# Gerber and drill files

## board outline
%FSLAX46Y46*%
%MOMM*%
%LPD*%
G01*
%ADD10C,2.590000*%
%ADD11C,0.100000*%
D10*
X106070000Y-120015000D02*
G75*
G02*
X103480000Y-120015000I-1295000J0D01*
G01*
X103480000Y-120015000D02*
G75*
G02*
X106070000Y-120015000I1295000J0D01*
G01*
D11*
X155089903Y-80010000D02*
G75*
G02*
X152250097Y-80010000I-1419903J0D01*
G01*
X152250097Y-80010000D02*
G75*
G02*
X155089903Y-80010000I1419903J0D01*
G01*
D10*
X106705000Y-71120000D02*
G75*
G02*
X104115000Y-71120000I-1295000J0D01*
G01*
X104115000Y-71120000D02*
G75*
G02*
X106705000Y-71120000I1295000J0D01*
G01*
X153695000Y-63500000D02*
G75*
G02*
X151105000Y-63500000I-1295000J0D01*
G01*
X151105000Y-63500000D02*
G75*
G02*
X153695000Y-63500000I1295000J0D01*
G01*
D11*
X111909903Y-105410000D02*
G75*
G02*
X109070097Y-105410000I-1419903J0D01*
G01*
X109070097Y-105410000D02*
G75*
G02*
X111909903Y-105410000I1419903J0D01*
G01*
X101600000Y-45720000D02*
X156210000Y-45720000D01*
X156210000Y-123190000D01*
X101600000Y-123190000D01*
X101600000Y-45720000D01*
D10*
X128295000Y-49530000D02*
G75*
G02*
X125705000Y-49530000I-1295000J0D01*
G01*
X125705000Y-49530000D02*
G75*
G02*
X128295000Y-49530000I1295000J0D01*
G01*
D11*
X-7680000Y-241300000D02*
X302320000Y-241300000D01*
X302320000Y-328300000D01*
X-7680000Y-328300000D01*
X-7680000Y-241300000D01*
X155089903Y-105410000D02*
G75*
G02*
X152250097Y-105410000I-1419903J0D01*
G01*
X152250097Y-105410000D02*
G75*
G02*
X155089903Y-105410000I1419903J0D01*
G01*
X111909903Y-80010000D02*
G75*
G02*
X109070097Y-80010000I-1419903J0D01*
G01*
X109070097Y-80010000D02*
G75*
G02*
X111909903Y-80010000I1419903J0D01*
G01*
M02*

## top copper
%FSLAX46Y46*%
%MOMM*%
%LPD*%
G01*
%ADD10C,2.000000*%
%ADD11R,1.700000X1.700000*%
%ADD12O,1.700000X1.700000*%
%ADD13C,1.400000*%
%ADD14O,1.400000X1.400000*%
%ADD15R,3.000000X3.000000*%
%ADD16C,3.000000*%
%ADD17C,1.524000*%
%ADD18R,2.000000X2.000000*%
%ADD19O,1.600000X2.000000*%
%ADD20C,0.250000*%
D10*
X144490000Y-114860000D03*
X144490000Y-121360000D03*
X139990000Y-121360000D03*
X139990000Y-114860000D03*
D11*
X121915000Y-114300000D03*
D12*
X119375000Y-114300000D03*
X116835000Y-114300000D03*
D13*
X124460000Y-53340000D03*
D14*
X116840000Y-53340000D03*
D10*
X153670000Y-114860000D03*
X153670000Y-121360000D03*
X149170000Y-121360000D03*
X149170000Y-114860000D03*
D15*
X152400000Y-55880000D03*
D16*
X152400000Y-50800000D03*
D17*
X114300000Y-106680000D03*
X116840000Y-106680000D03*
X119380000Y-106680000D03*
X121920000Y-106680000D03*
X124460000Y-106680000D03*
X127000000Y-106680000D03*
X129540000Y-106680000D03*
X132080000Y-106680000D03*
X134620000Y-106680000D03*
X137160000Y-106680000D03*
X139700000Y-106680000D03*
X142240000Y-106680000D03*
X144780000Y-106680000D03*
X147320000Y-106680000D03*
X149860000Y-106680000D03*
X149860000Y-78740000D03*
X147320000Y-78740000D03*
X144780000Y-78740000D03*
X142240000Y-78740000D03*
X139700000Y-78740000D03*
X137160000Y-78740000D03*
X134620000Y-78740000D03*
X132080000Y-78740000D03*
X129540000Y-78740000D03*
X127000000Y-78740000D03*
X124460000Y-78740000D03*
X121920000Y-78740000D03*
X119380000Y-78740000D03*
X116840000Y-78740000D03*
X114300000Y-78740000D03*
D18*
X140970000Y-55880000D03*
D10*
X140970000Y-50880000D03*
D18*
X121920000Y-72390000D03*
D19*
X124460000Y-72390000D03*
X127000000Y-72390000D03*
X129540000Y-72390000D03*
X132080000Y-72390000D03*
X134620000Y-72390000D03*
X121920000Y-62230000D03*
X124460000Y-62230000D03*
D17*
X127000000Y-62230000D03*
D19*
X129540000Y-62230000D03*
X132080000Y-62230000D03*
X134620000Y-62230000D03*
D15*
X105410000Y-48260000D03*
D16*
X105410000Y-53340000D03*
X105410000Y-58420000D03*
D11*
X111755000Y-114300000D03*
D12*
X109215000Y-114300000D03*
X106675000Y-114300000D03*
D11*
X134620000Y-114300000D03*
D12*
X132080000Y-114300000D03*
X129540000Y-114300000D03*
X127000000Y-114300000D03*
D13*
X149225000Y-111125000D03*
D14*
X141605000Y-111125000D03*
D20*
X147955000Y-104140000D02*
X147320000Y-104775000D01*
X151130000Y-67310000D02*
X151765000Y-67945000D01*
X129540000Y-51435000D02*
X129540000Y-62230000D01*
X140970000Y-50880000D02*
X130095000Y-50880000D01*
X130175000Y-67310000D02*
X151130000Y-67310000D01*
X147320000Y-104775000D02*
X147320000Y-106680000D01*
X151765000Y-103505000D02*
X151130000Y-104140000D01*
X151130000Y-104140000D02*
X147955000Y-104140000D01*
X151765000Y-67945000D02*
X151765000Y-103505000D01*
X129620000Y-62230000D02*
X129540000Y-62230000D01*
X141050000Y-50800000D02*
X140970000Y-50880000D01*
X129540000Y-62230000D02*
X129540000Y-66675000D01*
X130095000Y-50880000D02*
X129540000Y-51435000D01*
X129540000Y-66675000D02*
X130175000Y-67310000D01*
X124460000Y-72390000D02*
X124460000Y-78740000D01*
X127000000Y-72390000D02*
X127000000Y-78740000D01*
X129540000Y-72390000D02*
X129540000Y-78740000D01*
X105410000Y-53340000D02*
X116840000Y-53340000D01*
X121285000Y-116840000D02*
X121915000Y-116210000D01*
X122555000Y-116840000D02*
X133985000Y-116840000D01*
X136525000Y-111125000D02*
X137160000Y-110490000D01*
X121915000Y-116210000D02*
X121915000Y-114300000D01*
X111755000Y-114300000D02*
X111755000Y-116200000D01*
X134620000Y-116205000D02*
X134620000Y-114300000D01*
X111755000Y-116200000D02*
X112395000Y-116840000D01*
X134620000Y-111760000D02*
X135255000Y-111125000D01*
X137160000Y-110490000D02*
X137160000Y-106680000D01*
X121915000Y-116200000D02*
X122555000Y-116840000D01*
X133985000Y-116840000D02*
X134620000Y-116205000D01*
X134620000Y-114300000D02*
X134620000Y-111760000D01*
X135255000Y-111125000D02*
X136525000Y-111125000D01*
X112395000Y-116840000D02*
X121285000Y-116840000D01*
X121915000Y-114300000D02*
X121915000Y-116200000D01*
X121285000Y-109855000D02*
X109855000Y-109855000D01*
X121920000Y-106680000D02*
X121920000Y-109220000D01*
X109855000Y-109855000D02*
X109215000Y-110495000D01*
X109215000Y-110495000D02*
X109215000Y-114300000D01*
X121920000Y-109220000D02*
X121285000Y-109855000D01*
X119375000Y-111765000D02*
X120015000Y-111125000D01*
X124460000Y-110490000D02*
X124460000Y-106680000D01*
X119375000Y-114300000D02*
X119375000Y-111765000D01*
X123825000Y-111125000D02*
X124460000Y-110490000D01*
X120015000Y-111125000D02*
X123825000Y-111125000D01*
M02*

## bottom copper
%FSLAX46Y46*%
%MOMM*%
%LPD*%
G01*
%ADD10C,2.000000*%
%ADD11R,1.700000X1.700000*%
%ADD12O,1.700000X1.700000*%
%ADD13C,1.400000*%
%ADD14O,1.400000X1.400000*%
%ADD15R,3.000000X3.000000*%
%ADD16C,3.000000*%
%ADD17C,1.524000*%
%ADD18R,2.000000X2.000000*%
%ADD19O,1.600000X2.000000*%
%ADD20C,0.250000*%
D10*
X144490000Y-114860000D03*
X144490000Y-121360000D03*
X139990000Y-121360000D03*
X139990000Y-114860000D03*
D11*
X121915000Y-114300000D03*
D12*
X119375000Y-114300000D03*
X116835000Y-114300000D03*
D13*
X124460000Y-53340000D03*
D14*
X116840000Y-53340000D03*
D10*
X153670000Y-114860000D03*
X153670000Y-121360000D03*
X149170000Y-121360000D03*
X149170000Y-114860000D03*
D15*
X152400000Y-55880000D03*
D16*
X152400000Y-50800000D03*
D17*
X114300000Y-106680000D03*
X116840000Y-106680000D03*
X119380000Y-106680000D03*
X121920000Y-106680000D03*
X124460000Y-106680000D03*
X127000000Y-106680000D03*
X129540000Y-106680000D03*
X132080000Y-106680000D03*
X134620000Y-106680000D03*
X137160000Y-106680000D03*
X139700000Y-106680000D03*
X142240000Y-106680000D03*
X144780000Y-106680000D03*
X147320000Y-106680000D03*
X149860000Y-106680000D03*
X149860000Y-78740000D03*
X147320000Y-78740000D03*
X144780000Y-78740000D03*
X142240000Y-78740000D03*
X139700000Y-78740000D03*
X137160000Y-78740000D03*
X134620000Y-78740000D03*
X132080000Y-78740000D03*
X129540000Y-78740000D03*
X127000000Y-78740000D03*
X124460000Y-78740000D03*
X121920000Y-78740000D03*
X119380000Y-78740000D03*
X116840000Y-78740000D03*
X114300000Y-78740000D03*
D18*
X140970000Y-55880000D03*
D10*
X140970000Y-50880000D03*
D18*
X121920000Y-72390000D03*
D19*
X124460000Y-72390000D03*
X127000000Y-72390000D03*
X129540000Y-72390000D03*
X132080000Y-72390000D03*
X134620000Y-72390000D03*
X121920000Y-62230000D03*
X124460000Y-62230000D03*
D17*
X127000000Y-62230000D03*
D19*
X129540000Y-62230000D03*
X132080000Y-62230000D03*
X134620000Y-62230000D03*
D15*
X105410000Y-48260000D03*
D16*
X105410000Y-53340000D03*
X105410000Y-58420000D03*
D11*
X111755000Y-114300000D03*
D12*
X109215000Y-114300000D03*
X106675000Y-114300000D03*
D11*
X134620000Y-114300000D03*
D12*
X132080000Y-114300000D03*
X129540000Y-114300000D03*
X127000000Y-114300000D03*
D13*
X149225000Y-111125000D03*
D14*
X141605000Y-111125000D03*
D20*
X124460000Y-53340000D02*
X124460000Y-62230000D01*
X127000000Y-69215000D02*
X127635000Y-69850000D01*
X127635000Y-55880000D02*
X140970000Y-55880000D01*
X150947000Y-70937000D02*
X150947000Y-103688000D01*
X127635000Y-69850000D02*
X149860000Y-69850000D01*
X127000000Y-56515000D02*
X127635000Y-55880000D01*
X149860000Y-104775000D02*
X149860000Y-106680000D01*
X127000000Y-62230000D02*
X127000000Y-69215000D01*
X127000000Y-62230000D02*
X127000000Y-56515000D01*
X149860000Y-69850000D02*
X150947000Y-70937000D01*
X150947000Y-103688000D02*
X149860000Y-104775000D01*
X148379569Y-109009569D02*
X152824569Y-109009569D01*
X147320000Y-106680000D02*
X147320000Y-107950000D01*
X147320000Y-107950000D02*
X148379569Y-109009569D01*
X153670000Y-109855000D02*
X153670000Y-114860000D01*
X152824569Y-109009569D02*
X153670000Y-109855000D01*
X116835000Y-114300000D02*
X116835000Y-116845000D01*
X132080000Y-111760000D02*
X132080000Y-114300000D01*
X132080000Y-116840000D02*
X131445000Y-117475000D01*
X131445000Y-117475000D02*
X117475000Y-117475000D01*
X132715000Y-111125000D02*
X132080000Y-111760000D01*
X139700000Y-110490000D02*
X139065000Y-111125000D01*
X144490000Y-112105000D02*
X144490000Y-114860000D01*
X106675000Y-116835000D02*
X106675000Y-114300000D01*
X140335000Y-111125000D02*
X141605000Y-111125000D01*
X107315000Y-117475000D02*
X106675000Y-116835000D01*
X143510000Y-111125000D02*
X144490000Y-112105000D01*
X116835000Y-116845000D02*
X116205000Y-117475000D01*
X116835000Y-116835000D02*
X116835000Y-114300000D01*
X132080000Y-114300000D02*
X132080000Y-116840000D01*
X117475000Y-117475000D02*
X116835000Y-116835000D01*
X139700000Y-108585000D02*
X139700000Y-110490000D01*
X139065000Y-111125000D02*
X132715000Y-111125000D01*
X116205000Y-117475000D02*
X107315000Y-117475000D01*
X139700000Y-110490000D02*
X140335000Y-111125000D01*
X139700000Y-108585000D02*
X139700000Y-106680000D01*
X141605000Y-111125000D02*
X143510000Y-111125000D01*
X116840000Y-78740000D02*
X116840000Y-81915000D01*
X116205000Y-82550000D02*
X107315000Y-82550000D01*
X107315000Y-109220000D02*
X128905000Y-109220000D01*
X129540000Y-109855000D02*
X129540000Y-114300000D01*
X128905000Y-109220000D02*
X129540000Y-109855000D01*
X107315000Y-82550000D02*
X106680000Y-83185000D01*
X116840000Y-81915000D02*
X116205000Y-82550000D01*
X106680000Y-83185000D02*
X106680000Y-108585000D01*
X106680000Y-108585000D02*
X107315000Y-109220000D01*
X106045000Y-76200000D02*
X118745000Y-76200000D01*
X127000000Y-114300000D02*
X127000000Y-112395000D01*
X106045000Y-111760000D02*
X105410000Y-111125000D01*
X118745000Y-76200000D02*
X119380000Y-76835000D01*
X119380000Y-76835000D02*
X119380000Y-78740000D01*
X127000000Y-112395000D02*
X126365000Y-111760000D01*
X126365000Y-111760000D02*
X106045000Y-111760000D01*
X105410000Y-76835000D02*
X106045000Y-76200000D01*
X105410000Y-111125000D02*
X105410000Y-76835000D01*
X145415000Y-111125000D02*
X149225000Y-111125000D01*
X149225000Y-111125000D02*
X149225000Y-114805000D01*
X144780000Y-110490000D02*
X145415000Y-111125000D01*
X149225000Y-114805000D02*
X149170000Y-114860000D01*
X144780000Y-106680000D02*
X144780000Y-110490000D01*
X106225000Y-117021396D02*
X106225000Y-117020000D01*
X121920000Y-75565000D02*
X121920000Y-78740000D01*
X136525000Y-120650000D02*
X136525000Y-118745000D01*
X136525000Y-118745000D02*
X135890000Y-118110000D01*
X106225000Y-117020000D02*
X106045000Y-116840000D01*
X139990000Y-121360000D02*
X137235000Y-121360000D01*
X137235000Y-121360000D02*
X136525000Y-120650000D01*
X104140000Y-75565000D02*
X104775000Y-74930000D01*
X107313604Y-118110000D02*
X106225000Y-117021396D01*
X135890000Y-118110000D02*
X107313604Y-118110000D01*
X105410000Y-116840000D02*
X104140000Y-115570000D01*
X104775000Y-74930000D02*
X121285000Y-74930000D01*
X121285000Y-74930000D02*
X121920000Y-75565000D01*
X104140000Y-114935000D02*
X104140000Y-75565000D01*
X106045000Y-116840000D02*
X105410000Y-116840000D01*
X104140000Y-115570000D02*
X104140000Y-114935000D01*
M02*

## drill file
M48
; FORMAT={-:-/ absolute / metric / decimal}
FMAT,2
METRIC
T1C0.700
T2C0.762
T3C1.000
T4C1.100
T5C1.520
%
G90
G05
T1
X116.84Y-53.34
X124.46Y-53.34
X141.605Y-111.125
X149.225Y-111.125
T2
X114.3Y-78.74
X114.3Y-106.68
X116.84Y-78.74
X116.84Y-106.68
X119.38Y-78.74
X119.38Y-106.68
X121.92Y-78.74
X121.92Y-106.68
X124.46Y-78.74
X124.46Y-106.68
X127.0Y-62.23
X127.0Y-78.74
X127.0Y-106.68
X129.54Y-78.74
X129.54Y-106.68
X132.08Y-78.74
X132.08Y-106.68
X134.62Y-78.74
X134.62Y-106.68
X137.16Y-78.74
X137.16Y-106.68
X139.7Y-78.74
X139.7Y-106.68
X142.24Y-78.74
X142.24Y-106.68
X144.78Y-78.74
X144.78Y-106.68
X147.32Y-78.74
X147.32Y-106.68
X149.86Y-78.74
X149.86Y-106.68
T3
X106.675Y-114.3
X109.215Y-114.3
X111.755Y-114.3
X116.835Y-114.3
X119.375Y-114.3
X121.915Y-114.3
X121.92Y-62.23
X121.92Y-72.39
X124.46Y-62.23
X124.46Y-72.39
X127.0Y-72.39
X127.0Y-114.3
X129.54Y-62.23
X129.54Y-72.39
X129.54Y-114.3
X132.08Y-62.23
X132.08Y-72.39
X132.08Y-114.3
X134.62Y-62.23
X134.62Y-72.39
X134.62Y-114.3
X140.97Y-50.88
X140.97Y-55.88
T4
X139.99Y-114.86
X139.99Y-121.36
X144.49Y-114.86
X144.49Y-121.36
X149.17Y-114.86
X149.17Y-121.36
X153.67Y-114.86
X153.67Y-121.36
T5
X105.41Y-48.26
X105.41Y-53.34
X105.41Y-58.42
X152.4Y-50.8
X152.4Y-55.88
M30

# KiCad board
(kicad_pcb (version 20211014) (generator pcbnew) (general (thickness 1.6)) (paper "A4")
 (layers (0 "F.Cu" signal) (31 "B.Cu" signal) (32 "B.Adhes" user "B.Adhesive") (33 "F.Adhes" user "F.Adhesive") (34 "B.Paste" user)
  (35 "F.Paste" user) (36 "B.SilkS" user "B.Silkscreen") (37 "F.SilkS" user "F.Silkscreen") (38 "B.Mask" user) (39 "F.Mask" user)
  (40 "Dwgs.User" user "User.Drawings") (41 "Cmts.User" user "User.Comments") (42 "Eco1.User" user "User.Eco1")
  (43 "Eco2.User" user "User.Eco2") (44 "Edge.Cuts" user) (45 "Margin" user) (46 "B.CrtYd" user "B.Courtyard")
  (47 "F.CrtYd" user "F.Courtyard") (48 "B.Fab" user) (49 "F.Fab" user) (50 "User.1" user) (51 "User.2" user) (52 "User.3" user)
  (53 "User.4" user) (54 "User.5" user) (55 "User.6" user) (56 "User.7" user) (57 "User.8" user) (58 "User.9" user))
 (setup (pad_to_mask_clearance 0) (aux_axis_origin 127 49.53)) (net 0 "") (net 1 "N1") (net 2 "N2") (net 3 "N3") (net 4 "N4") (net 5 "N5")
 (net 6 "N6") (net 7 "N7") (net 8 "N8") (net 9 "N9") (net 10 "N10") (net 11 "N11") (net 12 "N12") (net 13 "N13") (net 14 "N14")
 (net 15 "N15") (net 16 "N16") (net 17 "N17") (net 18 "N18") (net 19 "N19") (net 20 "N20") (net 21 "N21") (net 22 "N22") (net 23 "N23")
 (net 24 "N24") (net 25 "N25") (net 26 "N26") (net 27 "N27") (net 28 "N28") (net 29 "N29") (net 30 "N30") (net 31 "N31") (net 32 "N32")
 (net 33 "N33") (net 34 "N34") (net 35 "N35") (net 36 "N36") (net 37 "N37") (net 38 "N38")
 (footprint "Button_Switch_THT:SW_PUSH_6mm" (layer "F.Cu") (at 144.49 114.86 -90)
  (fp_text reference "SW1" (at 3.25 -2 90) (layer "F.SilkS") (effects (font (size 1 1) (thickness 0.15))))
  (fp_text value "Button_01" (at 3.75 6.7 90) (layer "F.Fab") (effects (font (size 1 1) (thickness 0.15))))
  (pad "1" thru_hole circle (at 0 0) (size 2 2) (drill 1.1) (layers *.Cu *.Mask) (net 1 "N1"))
  (pad "1" thru_hole circle (at 6.5 0) (size 2 2) (drill 1.1) (layers *.Cu *.Mask) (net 1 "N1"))
  (pad "2" thru_hole circle (at 6.5 4.5) (size 2 2) (drill 1.1) (layers *.Cu *.Mask) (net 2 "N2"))
  (pad "2" thru_hole circle (at 0 4.5) (size 2 2) (drill 1.1) (layers *.Cu *.Mask) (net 2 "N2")))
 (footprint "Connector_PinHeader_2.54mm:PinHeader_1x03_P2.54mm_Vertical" (layer "F.Cu") (at 121.915 114.3 -90)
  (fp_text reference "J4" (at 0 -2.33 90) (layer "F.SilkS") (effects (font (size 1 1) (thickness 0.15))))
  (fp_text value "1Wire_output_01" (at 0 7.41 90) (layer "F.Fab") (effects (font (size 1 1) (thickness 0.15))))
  (pad "1" thru_hole rect (at 0 0 270) (size 1.7 1.7) (drill 1) (layers *.Cu *.Mask) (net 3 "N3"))
  (pad "2" thru_hole oval (at 0 2.54 270) (size 1.7 1.7) (drill 1) (layers *.Cu *.Mask) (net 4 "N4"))
  (pad "3" thru_hole oval (at 0 5.08 270) (size 1.7 1.7) (drill 1) (layers *.Cu *.Mask) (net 1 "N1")))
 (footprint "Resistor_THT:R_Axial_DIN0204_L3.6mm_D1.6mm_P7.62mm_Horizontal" (layer "F.Cu") (at 124.46 53.34 180)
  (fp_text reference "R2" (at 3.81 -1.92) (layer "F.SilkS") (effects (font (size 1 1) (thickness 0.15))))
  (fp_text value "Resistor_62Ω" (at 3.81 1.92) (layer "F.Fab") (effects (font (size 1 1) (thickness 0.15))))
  (pad "1" thru_hole circle (at 0 0 180) (size 1.4 1.4) (drill 0.7) (layers *.Cu *.Mask) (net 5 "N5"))
  (pad "2" thru_hole oval (at 7.62 0 180) (size 1.4 1.4) (drill 0.7) (layers *.Cu *.Mask) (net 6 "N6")))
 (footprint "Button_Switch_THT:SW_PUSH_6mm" (layer "F.Cu") (at 153.67 114.86 -90)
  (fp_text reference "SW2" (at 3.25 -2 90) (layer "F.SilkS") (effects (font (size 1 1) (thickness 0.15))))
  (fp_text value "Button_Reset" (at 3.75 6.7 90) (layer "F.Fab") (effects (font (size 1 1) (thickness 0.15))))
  (pad "1" thru_hole circle (at 0 0) (size 2 2) (drill 1.1) (layers *.Cu *.Mask) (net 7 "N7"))
  (pad "1" thru_hole circle (at 6.5 0) (size 2 2) (drill 1.1) (layers *.Cu *.Mask) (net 7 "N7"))
  (pad "2" thru_hole circle (at 6.5 4.5) (size 2 2) (drill 1.1) (layers *.Cu *.Mask) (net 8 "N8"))
  (pad "2" thru_hole circle (at 0 4.5) (size 2 2) (drill 1.1) (layers *.Cu *.Mask) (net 8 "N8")))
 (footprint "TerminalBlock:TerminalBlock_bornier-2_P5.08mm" (layer "F.Cu") (at 152.4 55.88 90)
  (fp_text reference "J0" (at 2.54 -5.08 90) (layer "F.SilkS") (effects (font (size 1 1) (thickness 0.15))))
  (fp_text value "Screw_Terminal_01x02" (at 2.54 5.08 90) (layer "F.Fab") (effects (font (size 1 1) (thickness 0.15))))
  (pad "1" thru_hole rect (at 0 0 90) (size 3 3) (drill 1.52) (layers *.Cu *.Mask) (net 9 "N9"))
  (pad "2" thru_hole circle (at 5.08 0 90) (size 3 3) (drill 1.52) (layers *.Cu *.Mask) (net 7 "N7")))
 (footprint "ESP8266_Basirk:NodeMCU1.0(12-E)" (layer "F.Cu") (at 132.08 92.71 90)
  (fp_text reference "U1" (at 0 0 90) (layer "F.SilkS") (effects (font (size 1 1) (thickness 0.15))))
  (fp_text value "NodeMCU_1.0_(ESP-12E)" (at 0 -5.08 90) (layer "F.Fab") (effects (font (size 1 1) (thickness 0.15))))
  (pad "1" thru_hole circle locked (at -13.97 -17.78 90) (size 1.524 1.524) (drill 0.762) (layers *.Cu *.Mask "F.SilkS") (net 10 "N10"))
  (pad "2" thru_hole circle locked (at -13.97 -15.24 90) (size 1.524 1.524) (drill 0.762) (layers *.Cu *.Mask "F.SilkS") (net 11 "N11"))
  (pad "3" thru_hole circle locked (at -13.97 -12.7 90) (size 1.524 1.524) (drill 0.762) (layers *.Cu *.Mask "F.SilkS") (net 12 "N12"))
  (pad "4" thru_hole circle locked (at -13.97 -10.16 90) (size 1.524 1.524) (drill 0.762) (layers *.Cu *.Mask "F.SilkS") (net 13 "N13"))
  (pad "5" thru_hole circle locked (at -13.97 -7.62 90) (size 1.524 1.524) (drill 0.762) (layers *.Cu *.Mask "F.SilkS") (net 4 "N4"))
  (pad "6" thru_hole circle locked (at -13.97 -5.08 90) (size 1.524 1.524) (drill 0.762) (layers *.Cu *.Mask "F.SilkS") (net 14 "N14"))
  (pad "7" thru_hole circle locked (at -13.97 -2.54 90) (size 1.524 1.524) (drill 0.762) (layers *.Cu *.Mask "F.SilkS") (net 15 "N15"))
  (pad "8" thru_hole circle locked (at -13.97 0 90) (size 1.524 1.524) (drill 0.762) (layers *.Cu *.Mask "F.SilkS") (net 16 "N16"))
  (pad "9" thru_hole circle locked (at -13.97 2.54 90) (size 1.524 1.524) (drill 0.762) (layers *.Cu *.Mask "F.SilkS") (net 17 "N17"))
  (pad "10" thru_hole circle locked (at -13.97 5.08 90) (size 1.524 1.524) (drill 0.762) (layers *.Cu *.Mask "F.SilkS") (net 3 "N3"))
  (pad "11" thru_hole circle locked (at -13.97 7.62 90) (size 1.524 1.524) (drill 0.762) (layers *.Cu *.Mask "F.SilkS") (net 1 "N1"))
  (pad "12" thru_hole circle locked (at -13.97 10.16 90) (size 1.524 1.524) (drill 0.762) (layers *.Cu *.Mask "F.SilkS") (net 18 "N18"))
  (pad "13" thru_hole circle locked (at -13.97 12.7 90) (size 1.524 1.524) (drill 0.762) (layers *.Cu *.Mask "F.SilkS") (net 8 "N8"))
  (pad "14" thru_hole circle locked (at -13.97 15.24 90) (size 1.524 1.524) (drill 0.762) (layers *.Cu *.Mask "F.SilkS") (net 7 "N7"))
  (pad "15" thru_hole circle locked (at -13.97 17.78 90) (size 1.524 1.524) (drill 0.762) (layers *.Cu *.Mask "F.SilkS") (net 9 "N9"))
  (pad "16" thru_hole circle locked (at 13.97 17.78 90) (size 1.524 1.524) (drill 0.762) (layers *.Cu *.Mask "F.SilkS") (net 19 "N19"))
  (pad "17" thru_hole circle locked (at 13.97 15.24 90) (size 1.524 1.524) (drill 0.762) (layers *.Cu *.Mask "F.SilkS") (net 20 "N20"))
  (pad "18" thru_hole circle locked (at 13.97 12.7 90) (size 1.524 1.524) (drill 0.762) (layers *.Cu *.Mask "F.SilkS") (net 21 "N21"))
  (pad "19" thru_hole circle locked (at 13.97 10.16 90) (size 1.524 1.524) (drill 0.762) (layers *.Cu *.Mask "F.SilkS") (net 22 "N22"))
  (pad "20" thru_hole circle locked (at 13.97 7.62 90) (size 1.524 1.524) (drill 0.762) (layers *.Cu *.Mask "F.SilkS") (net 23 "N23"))
  (pad "21" thru_hole circle locked (at 13.97 5.08 90) (size 1.524 1.524) (drill 0.762) (layers *.Cu *.Mask "F.SilkS") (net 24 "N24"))
  (pad "22" thru_hole circle locked (at 13.97 2.54 90) (size 1.524 1.524) (drill 0.762) (layers *.Cu *.Mask "F.SilkS") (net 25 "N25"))
  (pad "23" thru_hole circle locked (at 13.97 0 90) (size 1.524 1.524) (drill 0.762) (layers *.Cu *.Mask "F.SilkS") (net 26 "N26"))
  (pad "24" thru_hole circle locked (at 13.97 -2.54 90) (size 1.524 1.524) (drill 0.762) (layers *.Cu *.Mask "F.SilkS") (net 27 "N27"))
  (pad "25" thru_hole circle locked (at 13.97 -5.08 90) (size 1.524 1.524) (drill 0.762) (layers *.Cu *.Mask "F.SilkS") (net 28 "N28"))
  (pad "26" thru_hole circle locked (at 13.97 -7.62 90) (size 1.524 1.524) (drill 0.762) (layers *.Cu *.Mask "F.SilkS") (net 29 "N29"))
  (pad "27" thru_hole circle locked (at 13.97 -10.16 90) (size 1.524 1.524) (drill 0.762) (layers *.Cu *.Mask "F.SilkS") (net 2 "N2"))
  (pad "28" thru_hole circle locked (at 13.97 -12.7 90) (size 1.524 1.524) (drill 0.762) (layers *.Cu *.Mask "F.SilkS") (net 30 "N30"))
  (pad "29" thru_hole circle locked (at 13.97 -15.24 90) (size 1.524 1.524) (drill 0.762) (layers *.Cu *.Mask "F.SilkS") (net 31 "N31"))
  (pad "30" thru_hole circle locked (at 13.97 -17.78 90) (size 1.524 1.524) (drill 0.762) (layers *.Cu *.Mask "F.SilkS") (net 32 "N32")))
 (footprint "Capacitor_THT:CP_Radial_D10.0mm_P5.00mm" (layer "F.Cu") (at 140.97 55.88 90)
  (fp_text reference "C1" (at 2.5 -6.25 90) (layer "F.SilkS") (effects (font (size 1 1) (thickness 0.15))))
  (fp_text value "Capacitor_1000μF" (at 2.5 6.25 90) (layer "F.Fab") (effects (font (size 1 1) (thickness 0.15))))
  (pad "1" thru_hole rect (at 0 0 90) (size 2 2) (drill 1) (layers *.Cu *.Mask) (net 9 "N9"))
  (pad "2" thru_hole circle (at 5 0 90) (size 2 2) (drill 1) (layers *.Cu *.Mask) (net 7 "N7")))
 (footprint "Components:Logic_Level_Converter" (layer "F.Cu") (at 128.27 67.31 90)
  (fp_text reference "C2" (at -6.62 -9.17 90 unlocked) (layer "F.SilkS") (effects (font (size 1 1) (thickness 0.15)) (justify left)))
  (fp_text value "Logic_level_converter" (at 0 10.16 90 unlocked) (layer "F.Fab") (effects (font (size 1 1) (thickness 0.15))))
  (pad "1" thru_hole rect (at -5.08 -6.35 90) (size 2 2) (drill 1) (layers *.Cu *.Mask) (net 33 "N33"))
  (pad "2" thru_hole oval (at -5.08 -3.81 90) (size 2 1.6) (drill 1) (layers *.Cu *.Mask) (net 29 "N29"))
  (pad "3" thru_hole oval (at -5.08 -1.27 90) (size 2 1.6) (drill 1) (layers *.Cu *.Mask) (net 28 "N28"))
  (pad "4" thru_hole oval (at -5.08 1.27 90) (size 2 1.6) (drill 1) (layers *.Cu *.Mask) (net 27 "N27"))
  (pad "5" thru_hole oval (at -5.08 3.81 90) (size 2 1.6) (drill 1) (layers *.Cu *.Mask) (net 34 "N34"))
  (pad "6" thru_hole oval (at -5.08 6.35 90) (size 2 1.6) (drill 1) (layers *.Cu *.Mask) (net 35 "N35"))
  (pad "7" thru_hole oval (at 5.08 -6.35 90) (size 2 1.6) (drill 1) (layers *.Cu *.Mask) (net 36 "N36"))
  (pad "8" thru_hole oval (at 5.08 -3.81 90) (size 2 1.6) (drill 1) (layers *.Cu *.Mask) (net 5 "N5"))
  (pad "9" thru_hole circle (at 5.08 -1.27 90) (size 1.524 1.524) (drill 0.762) (layers *.Cu *.Mask) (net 9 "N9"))
  (pad "10" thru_hole oval (at 5.08 1.27 90) (size 2 1.6) (drill 1) (layers *.Cu *.Mask) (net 7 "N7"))
  (pad "11" thru_hole oval (at 5.08 3.81 90) (size 2 1.6) (drill 1) (layers *.Cu *.Mask) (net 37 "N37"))
  (pad "12" thru_hole oval (at 5.08 6.35 90) (size 2 1.6) (drill 1) (layers *.Cu *.Mask) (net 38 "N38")))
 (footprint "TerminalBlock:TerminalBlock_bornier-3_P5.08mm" (layer "F.Cu") (at 105.41 48.26 -90)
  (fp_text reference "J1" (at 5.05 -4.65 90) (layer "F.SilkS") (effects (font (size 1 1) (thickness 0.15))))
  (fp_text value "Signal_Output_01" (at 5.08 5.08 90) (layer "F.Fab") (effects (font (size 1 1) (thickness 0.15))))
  (pad "1" thru_hole rect (at 0 0 270) (size 3 3) (drill 1.52) (layers *.Cu *.Mask) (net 9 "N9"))
  (pad "2" thru_hole circle (at 5.08 0 270) (size 3 3) (drill 1.52) (layers *.Cu *.Mask) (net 6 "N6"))
  (pad "3" thru_hole circle (at 10.16 0 270) (size 3 3) (drill 1.52) (layers *.Cu *.Mask) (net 7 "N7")))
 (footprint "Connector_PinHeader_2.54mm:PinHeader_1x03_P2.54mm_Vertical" (layer "F.Cu") (at 111.755 114.3 -90)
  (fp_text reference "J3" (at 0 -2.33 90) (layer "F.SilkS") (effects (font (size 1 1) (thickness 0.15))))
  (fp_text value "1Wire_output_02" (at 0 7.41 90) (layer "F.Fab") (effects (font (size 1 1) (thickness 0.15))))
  (pad "1" thru_hole rect (at 0 0 270) (size 1.7 1.7) (drill 1) (layers *.Cu *.Mask) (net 3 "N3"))
  (pad "2" thru_hole oval (at 0 2.54 270) (size 1.7 1.7) (drill 1) (layers *.Cu *.Mask) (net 13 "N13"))
  (pad "3" thru_hole oval (at 0 5.08 270) (size 1.7 1.7) (drill 1) (layers *.Cu *.Mask) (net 1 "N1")))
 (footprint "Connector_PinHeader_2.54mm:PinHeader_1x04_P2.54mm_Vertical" (layer "F.Cu") (at 134.62 114.3 -90)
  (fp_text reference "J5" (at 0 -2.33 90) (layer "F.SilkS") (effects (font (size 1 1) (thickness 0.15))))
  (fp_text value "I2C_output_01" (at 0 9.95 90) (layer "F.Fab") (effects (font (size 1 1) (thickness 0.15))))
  (pad "1" thru_hole rect (at 0 0 270) (size 1.7 1.7) (drill 1) (layers *.Cu *.Mask) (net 3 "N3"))
  (pad "2" thru_hole oval (at 0 2.54 270) (size 1.7 1.7) (drill 1) (layers *.Cu *.Mask) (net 1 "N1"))
  (pad "3" thru_hole oval (at 0 5.08 270) (size 1.7 1.7) (drill 1) (layers *.Cu *.Mask) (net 31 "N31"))
  (pad "4" thru_hole oval (at 0 7.62 270) (size 1.7 1.7) (drill 1) (layers *.Cu *.Mask) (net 30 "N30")))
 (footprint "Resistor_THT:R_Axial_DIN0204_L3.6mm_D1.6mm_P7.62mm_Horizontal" (layer "F.Cu") (at 149.225 111.125 180)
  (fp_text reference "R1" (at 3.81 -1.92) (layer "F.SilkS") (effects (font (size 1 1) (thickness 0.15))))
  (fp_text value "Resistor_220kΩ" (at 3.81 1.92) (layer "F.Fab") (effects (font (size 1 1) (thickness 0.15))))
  (pad "1" thru_hole circle (at 0 0 180) (size 1.4 1.4) (drill 0.7) (layers *.Cu *.Mask) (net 8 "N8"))
  (pad "2" thru_hole oval (at 7.62 0 180) (size 1.4 1.4) (drill 0.7) (layers *.Cu *.Mask) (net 1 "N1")))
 (gr_circle (center 104.775 120.015) (end 107.315 120.015) (layer "Edge.Cuts") (width 0.1) (fill solid))
 (gr_circle (center 153.67 80.01) (end 154.94 80.645) (layer "Edge.Cuts") (width 0.1) (fill none))
 (gr_circle (center 105.41 71.12) (end 107.95 71.12) (layer "Edge.Cuts") (width 0.1) (fill solid))
 (gr_circle (center 152.4 63.5) (end 154.94 63.5) (layer "Edge.Cuts") (width 0.1) (fill solid))
 (gr_circle (center 110.49 105.41) (end 111.76 106.045) (layer "Edge.Cuts") (width 0.1) (fill none))
 (gr_rect (start 101.6 45.72) (end 156.21 123.19) (layer "Edge.Cuts") (width 0.1) (fill none))
 (gr_circle (center 127 49.53) (end 129.54 49.53) (layer "Edge.Cuts") (width 0.1) (fill solid))
 (gr_rect (start -7.68 328.3) (end 302.32 241.3) (layer "Edge.Cuts") (width 0.1) (fill none))
 (gr_circle (center 153.67 105.41) (end 154.94 106.045) (layer "Edge.Cuts") (width 0.1) (fill none))
 (gr_circle (center 110.49 80.01) (end 111.76 80.645) (layer "Edge.Cuts") (width 0.1) (fill none))
 (segment (start 124.46 53.34) (end 124.46 62.23) (width 0.25) (layer "B.Cu") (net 5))
 (segment (start 127 69.215) (end 127.635 69.85) (width 0.25) (layer "B.Cu") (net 9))
 (segment (start 127.635 55.88) (end 140.97 55.88) (width 0.25) (layer "B.Cu") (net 9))
 (segment (start 150.947 70.937) (end 150.947 103.688) (width 0.25) (layer "B.Cu") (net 9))
 (segment (start 127.635 69.85) (end 149.86 69.85) (width 0.25) (layer "B.Cu") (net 9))
 (segment (start 127 56.515) (end 127.635 55.88) (width 0.25) (layer "B.Cu") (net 9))
 (segment (start 149.86 104.775) (end 149.86 106.68) (width 0.25) (layer "B.Cu") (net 9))
 (segment (start 127 62.23) (end 127 69.215) (width 0.25) (layer "B.Cu") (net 9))
 (segment (start 127 62.23) (end 127 56.515) (width 0.25) (layer "B.Cu") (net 9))
 (segment (start 149.86 69.85) (end 150.947 70.937) (width 0.25) (layer "B.Cu") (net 9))
 (segment (start 150.947 103.688) (end 149.86 104.775) (width 0.25) (layer "B.Cu") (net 9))
 (segment (start 147.955 104.14) (end 147.32 104.775) (width 0.25) (layer "F.Cu") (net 7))
 (segment (start 151.13 67.31) (end 151.765 67.945) (width 0.25) (layer "F.Cu") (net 7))
 (segment (start 129.54 51.435) (end 129.54 62.23) (width 0.25) (layer "F.Cu") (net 7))
 (segment (start 140.97 50.88) (end 130.095 50.88) (width 0.25) (layer "F.Cu") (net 7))
 (segment (start 130.175 67.31) (end 151.13 67.31) (width 0.25) (layer "F.Cu") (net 7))
 (segment (start 147.32 104.775) (end 147.32 106.68) (width 0.25) (layer "F.Cu") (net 7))
 (segment (start 151.765 103.505) (end 151.13 104.14) (width 0.25) (layer "F.Cu") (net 7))
 (segment (start 151.13 104.14) (end 147.955 104.14) (width 0.25) (layer "F.Cu") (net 7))
 (segment (start 151.765 67.945) (end 151.765 103.505) (width 0.25) (layer "F.Cu") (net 7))
 (segment (start 129.62 62.23) (end 129.54 62.23) (width 0.25) (layer "F.Cu") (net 7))
 (segment (start 141.05 50.8) (end 140.97 50.88) (width 0.25) (layer "F.Cu") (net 7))
 (segment (start 129.54 62.23) (end 129.54 66.675) (width 0.25) (layer "F.Cu") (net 7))
 (segment (start 130.095 50.88) (end 129.54 51.435) (width 0.25) (layer "F.Cu") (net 7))
 (segment (start 129.54 66.675) (end 130.175 67.31) (width 0.25) (layer "F.Cu") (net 7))
 (segment (start 148.379569 109.009569) (end 152.824569 109.009569) (width 0.25) (layer "B.Cu") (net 7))
 (segment (start 147.32 106.68) (end 147.32 107.95) (width 0.25) (layer "B.Cu") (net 7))
 (segment (start 147.32 107.95) (end 148.379569 109.009569) (width 0.25) (layer "B.Cu") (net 7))
 (segment (start 153.67 109.855) (end 153.67 114.86) (width 0.25) (layer "B.Cu") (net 7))
 (segment (start 152.824569 109.009569) (end 153.67 109.855) (width 0.25) (layer "B.Cu") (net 7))
 (segment (start 124.46 72.39) (end 124.46 78.74) (width 0.25) (layer "F.Cu") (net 29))
 (segment (start 127 72.39) (end 127 78.74) (width 0.25) (layer "F.Cu") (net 28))
 (segment (start 129.54 72.39) (end 129.54 78.74) (width 0.25) (layer "F.Cu") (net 27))
 (segment (start 105.41 53.34) (end 116.84 53.34) (width 0.25) (layer "F.Cu") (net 6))
 (segment (start 121.285 116.84) (end 121.915 116.21) (width 0.25) (layer "F.Cu") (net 3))
 (segment (start 122.555 116.84) (end 133.985 116.84) (width 0.25) (layer "F.Cu") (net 3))
 (segment (start 136.525 111.125) (end 137.16 110.49) (width 0.25) (layer "F.Cu") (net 3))
 (segment (start 121.915 116.21) (end 121.915 114.3) (width 0.25) (layer "F.Cu") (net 3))
 (segment (start 111.755 114.3) (end 111.755 116.2) (width 0.25) (layer "F.Cu") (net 3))
 (segment (start 134.62 116.205) (end 134.62 114.3) (width 0.25) (layer "F.Cu") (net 3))
 (segment (start 111.755 116.2) (end 112.395 116.84) (width 0.25) (layer "F.Cu") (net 3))
 (segment (start 134.62 111.76) (end 135.255 111.125) (width 0.25) (layer "F.Cu") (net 3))
 (segment (start 137.16 110.49) (end 137.16 106.68) (width 0.25) (layer "F.Cu") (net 3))
 (segment (start 121.915 116.2) (end 122.555 116.84) (width 0.25) (layer "F.Cu") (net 3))
 (segment (start 133.985 116.84) (end 134.62 116.205) (width 0.25) (layer "F.Cu") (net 3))
 (segment (start 134.62 114.3) (end 134.62 111.76) (width 0.25) (layer "F.Cu") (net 3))
 (segment (start 135.255 111.125) (end 136.525 111.125) (width 0.25) (layer "F.Cu") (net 3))
 (segment (start 112.395 116.84) (end 121.285 116.84) (width 0.25) (layer "F.Cu") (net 3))
 (segment (start 121.915 114.3) (end 121.915 116.2) (width 0.25) (layer "F.Cu") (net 3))
 (segment (start 121.285 109.855) (end 109.855 109.855) (width 0.25) (layer "F.Cu") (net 13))
 (segment (start 121.92 106.68) (end 121.92 109.22) (width 0.25) (layer "F.Cu") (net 13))
 (segment (start 109.855 109.855) (end 109.215 110.495) (width 0.25) (layer "F.Cu") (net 13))
 (segment (start 109.215 110.495) (end 109.215 114.3) (width 0.25) (layer "F.Cu") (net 13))
 (segment (start 121.92 109.22) (end 121.285 109.855) (width 0.25) (layer "F.Cu") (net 13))
 (segment (start 116.835 114.3) (end 116.835 116.845) (width 0.25) (layer "B.Cu") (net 1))
 (segment (start 132.08 111.76) (end 132.08 114.3) (width 0.25) (layer "B.Cu") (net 1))
 (segment (start 132.08 116.84) (end 131.445 117.475) (width 0.25) (layer "B.Cu") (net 1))
 (segment (start 131.445 117.475) (end 117.475 117.475) (width 0.25) (layer "B.Cu") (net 1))
 (segment (start 132.715 111.125) (end 132.08 111.76) (width 0.25) (layer "B.Cu") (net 1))
 (segment (start 139.7 110.49) (end 139.065 111.125) (width 0.25) (layer "B.Cu") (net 1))
 (segment (start 144.49 112.105) (end 144.49 114.86) (width 0.25) (layer "B.Cu") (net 1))
 (segment (start 106.675 116.835) (end 106.675 114.3) (width 0.25) (layer "B.Cu") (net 1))
 (segment (start 140.335 111.125) (end 141.605 111.125) (width 0.25) (layer "B.Cu") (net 1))
 (segment (start 107.315 117.475) (end 106.675 116.835) (width 0.25) (layer "B.Cu") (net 1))
 (segment (start 143.51 111.125) (end 144.49 112.105) (width 0.25) (layer "B.Cu") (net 1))
 (segment (start 116.835 116.845) (end 116.205 117.475) (width 0.25) (layer "B.Cu") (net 1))
 (segment (start 116.835 116.835) (end 116.835 114.3) (width 0.25) (layer "B.Cu") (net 1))
 (segment (start 132.08 114.3) (end 132.08 116.84) (width 0.25) (layer "B.Cu") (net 1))
 (segment (start 117.475 117.475) (end 116.835 116.835) (width 0.25) (layer "B.Cu") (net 1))
 (segment (start 139.7 108.585) (end 139.7 110.49) (width 0.25) (layer "B.Cu") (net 1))
 (segment (start 139.065 111.125) (end 132.715 111.125) (width 0.25) (layer "B.Cu") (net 1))
 (segment (start 116.205 117.475) (end 107.315 117.475) (width 0.25) (layer "B.Cu") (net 1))
 (segment (start 139.7 110.49) (end 140.335 111.125) (width 0.25) (layer "B.Cu") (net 1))
 (segment (start 139.7 108.585) (end 139.7 106.68) (width 0.25) (layer "B.Cu") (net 1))
 (segment (start 141.605 111.125) (end 143.51 111.125) (width 0.25) (layer "B.Cu") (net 1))
 (segment (start 119.375 111.765) (end 120.015 111.125) (width 0.25) (layer "F.Cu") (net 4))
 (segment (start 124.46 110.49) (end 124.46 106.68) (width 0.25) (layer "F.Cu") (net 4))
 (segment (start 119.375 114.3) (end 119.375 111.765) (width 0.25) (layer "F.Cu") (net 4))
 (segment (start 123.825 111.125) (end 124.46 110.49) (width 0.25) (layer "F.Cu") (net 4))
 (segment (start 120.015 111.125) (end 123.825 111.125) (width 0.25) (layer "F.Cu") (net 4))
 (segment (start 116.84 78.74) (end 116.84 81.915) (width 0.25) (layer "B.Cu") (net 31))
 (segment (start 116.205 82.55) (end 107.315 82.55) (width 0.25) (layer "B.Cu") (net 31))
 (segment (start 107.315 109.22) (end 128.905 109.22) (width 0.25) (layer "B.Cu") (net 31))
 (segment (start 129.54 109.855) (end 129.54 114.3) (width 0.25) (layer "B.Cu") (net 31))
 (segment (start 128.905 109.22) (end 129.54 109.855) (width 0.25) (layer "B.Cu") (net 31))
 (segment (start 107.315 82.55) (end 106.68 83.185) (width 0.25) (layer "B.Cu") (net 31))
 (segment (start 116.84 81.915) (end 116.205 82.55) (width 0.25) (layer "B.Cu") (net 31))
 (segment (start 106.68 83.185) (end 106.68 108.585) (width 0.25) (layer "B.Cu") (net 31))
 (segment (start 106.68 108.585) (end 107.315 109.22) (width 0.25) (layer "B.Cu") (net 31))
 (segment (start 106.045 76.2) (end 118.745 76.2) (width 0.25) (layer "B.Cu") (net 30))
 (segment (start 127 114.3) (end 127 112.395) (width 0.25) (layer "B.Cu") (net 30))
 (segment (start 106.045 111.76) (end 105.41 111.125) (width 0.25) (layer "B.Cu") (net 30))
 (segment (start 118.745 76.2) (end 119.38 76.835) (width 0.25) (layer "B.Cu") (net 30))
 (segment (start 119.38 76.835) (end 119.38 78.74) (width 0.25) (layer "B.Cu") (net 30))
 (segment (start 127 112.395) (end 126.365 111.76) (width 0.25) (layer "B.Cu") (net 30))
 (segment (start 126.365 111.76) (end 106.045 111.76) (width 0.25) (layer "B.Cu") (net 30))
 (segment (start 105.41 76.835) (end 106.045 76.2) (width 0.25) (layer "B.Cu") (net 30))
 (segment (start 105.41 111.125) (end 105.41 76.835) (width 0.25) (layer "B.Cu") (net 30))
 (segment (start 145.415 111.125) (end 149.225 111.125) (width 0.25) (layer "B.Cu") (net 8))
 (segment (start 149.225 111.125) (end 149.225 114.805) (width 0.25) (layer "B.Cu") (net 8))
 (segment (start 144.78 110.49) (end 145.415 111.125) (width 0.25) (layer "B.Cu") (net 8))
 (segment (start 149.225 114.805) (end 149.17 114.86) (width 0.25) (layer "B.Cu") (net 8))
 (segment (start 144.78 106.68) (end 144.78 110.49) (width 0.25) (layer "B.Cu") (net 8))
 (segment (start 106.225 117.021396) (end 106.225 117.02) (width 0.25) (layer "B.Cu") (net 2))
 (segment (start 121.92 75.565) (end 121.92 78.74) (width 0.25) (layer "B.Cu") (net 2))
 (segment (start 136.525 120.65) (end 136.525 118.745) (width 0.25) (layer "B.Cu") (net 2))
 (segment (start 136.525 118.745) (end 135.89 118.11) (width 0.25) (layer "B.Cu") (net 2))
 (segment (start 106.225 117.02) (end 106.045 116.84) (width 0.25) (layer "B.Cu") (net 2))
 (segment (start 139.99 121.36) (end 137.235 121.36) (width 0.25) (layer "B.Cu") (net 2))
 (segment (start 137.235 121.36) (end 136.525 120.65) (width 0.25) (layer "B.Cu") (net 2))
 (segment (start 104.14 75.565) (end 104.775 74.93) (width 0.25) (layer "B.Cu") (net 2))
 (segment (start 107.313604 118.11) (end 106.225 117.021396) (width 0.25) (layer "B.Cu") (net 2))
 (segment (start 135.89 118.11) (end 107.313604 118.11) (width 0.25) (layer "B.Cu") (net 2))
 (segment (start 105.41 116.84) (end 104.14 115.57) (width 0.25) (layer "B.Cu") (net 2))
 (segment (start 104.775 74.93) (end 121.285 74.93) (width 0.25) (layer "B.Cu") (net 2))
 (segment (start 121.285 74.93) (end 121.92 75.565) (width 0.25) (layer "B.Cu") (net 2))
 (segment (start 104.14 114.935) (end 104.14 75.565) (width 0.25) (layer "B.Cu") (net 2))
 (segment (start 106.045 116.84) (end 105.41 116.84) (width 0.25) (layer "B.Cu") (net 2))
 (segment (start 104.14 115.57) (end 104.14 114.935) (width 0.25) (layer "B.Cu") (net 2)))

